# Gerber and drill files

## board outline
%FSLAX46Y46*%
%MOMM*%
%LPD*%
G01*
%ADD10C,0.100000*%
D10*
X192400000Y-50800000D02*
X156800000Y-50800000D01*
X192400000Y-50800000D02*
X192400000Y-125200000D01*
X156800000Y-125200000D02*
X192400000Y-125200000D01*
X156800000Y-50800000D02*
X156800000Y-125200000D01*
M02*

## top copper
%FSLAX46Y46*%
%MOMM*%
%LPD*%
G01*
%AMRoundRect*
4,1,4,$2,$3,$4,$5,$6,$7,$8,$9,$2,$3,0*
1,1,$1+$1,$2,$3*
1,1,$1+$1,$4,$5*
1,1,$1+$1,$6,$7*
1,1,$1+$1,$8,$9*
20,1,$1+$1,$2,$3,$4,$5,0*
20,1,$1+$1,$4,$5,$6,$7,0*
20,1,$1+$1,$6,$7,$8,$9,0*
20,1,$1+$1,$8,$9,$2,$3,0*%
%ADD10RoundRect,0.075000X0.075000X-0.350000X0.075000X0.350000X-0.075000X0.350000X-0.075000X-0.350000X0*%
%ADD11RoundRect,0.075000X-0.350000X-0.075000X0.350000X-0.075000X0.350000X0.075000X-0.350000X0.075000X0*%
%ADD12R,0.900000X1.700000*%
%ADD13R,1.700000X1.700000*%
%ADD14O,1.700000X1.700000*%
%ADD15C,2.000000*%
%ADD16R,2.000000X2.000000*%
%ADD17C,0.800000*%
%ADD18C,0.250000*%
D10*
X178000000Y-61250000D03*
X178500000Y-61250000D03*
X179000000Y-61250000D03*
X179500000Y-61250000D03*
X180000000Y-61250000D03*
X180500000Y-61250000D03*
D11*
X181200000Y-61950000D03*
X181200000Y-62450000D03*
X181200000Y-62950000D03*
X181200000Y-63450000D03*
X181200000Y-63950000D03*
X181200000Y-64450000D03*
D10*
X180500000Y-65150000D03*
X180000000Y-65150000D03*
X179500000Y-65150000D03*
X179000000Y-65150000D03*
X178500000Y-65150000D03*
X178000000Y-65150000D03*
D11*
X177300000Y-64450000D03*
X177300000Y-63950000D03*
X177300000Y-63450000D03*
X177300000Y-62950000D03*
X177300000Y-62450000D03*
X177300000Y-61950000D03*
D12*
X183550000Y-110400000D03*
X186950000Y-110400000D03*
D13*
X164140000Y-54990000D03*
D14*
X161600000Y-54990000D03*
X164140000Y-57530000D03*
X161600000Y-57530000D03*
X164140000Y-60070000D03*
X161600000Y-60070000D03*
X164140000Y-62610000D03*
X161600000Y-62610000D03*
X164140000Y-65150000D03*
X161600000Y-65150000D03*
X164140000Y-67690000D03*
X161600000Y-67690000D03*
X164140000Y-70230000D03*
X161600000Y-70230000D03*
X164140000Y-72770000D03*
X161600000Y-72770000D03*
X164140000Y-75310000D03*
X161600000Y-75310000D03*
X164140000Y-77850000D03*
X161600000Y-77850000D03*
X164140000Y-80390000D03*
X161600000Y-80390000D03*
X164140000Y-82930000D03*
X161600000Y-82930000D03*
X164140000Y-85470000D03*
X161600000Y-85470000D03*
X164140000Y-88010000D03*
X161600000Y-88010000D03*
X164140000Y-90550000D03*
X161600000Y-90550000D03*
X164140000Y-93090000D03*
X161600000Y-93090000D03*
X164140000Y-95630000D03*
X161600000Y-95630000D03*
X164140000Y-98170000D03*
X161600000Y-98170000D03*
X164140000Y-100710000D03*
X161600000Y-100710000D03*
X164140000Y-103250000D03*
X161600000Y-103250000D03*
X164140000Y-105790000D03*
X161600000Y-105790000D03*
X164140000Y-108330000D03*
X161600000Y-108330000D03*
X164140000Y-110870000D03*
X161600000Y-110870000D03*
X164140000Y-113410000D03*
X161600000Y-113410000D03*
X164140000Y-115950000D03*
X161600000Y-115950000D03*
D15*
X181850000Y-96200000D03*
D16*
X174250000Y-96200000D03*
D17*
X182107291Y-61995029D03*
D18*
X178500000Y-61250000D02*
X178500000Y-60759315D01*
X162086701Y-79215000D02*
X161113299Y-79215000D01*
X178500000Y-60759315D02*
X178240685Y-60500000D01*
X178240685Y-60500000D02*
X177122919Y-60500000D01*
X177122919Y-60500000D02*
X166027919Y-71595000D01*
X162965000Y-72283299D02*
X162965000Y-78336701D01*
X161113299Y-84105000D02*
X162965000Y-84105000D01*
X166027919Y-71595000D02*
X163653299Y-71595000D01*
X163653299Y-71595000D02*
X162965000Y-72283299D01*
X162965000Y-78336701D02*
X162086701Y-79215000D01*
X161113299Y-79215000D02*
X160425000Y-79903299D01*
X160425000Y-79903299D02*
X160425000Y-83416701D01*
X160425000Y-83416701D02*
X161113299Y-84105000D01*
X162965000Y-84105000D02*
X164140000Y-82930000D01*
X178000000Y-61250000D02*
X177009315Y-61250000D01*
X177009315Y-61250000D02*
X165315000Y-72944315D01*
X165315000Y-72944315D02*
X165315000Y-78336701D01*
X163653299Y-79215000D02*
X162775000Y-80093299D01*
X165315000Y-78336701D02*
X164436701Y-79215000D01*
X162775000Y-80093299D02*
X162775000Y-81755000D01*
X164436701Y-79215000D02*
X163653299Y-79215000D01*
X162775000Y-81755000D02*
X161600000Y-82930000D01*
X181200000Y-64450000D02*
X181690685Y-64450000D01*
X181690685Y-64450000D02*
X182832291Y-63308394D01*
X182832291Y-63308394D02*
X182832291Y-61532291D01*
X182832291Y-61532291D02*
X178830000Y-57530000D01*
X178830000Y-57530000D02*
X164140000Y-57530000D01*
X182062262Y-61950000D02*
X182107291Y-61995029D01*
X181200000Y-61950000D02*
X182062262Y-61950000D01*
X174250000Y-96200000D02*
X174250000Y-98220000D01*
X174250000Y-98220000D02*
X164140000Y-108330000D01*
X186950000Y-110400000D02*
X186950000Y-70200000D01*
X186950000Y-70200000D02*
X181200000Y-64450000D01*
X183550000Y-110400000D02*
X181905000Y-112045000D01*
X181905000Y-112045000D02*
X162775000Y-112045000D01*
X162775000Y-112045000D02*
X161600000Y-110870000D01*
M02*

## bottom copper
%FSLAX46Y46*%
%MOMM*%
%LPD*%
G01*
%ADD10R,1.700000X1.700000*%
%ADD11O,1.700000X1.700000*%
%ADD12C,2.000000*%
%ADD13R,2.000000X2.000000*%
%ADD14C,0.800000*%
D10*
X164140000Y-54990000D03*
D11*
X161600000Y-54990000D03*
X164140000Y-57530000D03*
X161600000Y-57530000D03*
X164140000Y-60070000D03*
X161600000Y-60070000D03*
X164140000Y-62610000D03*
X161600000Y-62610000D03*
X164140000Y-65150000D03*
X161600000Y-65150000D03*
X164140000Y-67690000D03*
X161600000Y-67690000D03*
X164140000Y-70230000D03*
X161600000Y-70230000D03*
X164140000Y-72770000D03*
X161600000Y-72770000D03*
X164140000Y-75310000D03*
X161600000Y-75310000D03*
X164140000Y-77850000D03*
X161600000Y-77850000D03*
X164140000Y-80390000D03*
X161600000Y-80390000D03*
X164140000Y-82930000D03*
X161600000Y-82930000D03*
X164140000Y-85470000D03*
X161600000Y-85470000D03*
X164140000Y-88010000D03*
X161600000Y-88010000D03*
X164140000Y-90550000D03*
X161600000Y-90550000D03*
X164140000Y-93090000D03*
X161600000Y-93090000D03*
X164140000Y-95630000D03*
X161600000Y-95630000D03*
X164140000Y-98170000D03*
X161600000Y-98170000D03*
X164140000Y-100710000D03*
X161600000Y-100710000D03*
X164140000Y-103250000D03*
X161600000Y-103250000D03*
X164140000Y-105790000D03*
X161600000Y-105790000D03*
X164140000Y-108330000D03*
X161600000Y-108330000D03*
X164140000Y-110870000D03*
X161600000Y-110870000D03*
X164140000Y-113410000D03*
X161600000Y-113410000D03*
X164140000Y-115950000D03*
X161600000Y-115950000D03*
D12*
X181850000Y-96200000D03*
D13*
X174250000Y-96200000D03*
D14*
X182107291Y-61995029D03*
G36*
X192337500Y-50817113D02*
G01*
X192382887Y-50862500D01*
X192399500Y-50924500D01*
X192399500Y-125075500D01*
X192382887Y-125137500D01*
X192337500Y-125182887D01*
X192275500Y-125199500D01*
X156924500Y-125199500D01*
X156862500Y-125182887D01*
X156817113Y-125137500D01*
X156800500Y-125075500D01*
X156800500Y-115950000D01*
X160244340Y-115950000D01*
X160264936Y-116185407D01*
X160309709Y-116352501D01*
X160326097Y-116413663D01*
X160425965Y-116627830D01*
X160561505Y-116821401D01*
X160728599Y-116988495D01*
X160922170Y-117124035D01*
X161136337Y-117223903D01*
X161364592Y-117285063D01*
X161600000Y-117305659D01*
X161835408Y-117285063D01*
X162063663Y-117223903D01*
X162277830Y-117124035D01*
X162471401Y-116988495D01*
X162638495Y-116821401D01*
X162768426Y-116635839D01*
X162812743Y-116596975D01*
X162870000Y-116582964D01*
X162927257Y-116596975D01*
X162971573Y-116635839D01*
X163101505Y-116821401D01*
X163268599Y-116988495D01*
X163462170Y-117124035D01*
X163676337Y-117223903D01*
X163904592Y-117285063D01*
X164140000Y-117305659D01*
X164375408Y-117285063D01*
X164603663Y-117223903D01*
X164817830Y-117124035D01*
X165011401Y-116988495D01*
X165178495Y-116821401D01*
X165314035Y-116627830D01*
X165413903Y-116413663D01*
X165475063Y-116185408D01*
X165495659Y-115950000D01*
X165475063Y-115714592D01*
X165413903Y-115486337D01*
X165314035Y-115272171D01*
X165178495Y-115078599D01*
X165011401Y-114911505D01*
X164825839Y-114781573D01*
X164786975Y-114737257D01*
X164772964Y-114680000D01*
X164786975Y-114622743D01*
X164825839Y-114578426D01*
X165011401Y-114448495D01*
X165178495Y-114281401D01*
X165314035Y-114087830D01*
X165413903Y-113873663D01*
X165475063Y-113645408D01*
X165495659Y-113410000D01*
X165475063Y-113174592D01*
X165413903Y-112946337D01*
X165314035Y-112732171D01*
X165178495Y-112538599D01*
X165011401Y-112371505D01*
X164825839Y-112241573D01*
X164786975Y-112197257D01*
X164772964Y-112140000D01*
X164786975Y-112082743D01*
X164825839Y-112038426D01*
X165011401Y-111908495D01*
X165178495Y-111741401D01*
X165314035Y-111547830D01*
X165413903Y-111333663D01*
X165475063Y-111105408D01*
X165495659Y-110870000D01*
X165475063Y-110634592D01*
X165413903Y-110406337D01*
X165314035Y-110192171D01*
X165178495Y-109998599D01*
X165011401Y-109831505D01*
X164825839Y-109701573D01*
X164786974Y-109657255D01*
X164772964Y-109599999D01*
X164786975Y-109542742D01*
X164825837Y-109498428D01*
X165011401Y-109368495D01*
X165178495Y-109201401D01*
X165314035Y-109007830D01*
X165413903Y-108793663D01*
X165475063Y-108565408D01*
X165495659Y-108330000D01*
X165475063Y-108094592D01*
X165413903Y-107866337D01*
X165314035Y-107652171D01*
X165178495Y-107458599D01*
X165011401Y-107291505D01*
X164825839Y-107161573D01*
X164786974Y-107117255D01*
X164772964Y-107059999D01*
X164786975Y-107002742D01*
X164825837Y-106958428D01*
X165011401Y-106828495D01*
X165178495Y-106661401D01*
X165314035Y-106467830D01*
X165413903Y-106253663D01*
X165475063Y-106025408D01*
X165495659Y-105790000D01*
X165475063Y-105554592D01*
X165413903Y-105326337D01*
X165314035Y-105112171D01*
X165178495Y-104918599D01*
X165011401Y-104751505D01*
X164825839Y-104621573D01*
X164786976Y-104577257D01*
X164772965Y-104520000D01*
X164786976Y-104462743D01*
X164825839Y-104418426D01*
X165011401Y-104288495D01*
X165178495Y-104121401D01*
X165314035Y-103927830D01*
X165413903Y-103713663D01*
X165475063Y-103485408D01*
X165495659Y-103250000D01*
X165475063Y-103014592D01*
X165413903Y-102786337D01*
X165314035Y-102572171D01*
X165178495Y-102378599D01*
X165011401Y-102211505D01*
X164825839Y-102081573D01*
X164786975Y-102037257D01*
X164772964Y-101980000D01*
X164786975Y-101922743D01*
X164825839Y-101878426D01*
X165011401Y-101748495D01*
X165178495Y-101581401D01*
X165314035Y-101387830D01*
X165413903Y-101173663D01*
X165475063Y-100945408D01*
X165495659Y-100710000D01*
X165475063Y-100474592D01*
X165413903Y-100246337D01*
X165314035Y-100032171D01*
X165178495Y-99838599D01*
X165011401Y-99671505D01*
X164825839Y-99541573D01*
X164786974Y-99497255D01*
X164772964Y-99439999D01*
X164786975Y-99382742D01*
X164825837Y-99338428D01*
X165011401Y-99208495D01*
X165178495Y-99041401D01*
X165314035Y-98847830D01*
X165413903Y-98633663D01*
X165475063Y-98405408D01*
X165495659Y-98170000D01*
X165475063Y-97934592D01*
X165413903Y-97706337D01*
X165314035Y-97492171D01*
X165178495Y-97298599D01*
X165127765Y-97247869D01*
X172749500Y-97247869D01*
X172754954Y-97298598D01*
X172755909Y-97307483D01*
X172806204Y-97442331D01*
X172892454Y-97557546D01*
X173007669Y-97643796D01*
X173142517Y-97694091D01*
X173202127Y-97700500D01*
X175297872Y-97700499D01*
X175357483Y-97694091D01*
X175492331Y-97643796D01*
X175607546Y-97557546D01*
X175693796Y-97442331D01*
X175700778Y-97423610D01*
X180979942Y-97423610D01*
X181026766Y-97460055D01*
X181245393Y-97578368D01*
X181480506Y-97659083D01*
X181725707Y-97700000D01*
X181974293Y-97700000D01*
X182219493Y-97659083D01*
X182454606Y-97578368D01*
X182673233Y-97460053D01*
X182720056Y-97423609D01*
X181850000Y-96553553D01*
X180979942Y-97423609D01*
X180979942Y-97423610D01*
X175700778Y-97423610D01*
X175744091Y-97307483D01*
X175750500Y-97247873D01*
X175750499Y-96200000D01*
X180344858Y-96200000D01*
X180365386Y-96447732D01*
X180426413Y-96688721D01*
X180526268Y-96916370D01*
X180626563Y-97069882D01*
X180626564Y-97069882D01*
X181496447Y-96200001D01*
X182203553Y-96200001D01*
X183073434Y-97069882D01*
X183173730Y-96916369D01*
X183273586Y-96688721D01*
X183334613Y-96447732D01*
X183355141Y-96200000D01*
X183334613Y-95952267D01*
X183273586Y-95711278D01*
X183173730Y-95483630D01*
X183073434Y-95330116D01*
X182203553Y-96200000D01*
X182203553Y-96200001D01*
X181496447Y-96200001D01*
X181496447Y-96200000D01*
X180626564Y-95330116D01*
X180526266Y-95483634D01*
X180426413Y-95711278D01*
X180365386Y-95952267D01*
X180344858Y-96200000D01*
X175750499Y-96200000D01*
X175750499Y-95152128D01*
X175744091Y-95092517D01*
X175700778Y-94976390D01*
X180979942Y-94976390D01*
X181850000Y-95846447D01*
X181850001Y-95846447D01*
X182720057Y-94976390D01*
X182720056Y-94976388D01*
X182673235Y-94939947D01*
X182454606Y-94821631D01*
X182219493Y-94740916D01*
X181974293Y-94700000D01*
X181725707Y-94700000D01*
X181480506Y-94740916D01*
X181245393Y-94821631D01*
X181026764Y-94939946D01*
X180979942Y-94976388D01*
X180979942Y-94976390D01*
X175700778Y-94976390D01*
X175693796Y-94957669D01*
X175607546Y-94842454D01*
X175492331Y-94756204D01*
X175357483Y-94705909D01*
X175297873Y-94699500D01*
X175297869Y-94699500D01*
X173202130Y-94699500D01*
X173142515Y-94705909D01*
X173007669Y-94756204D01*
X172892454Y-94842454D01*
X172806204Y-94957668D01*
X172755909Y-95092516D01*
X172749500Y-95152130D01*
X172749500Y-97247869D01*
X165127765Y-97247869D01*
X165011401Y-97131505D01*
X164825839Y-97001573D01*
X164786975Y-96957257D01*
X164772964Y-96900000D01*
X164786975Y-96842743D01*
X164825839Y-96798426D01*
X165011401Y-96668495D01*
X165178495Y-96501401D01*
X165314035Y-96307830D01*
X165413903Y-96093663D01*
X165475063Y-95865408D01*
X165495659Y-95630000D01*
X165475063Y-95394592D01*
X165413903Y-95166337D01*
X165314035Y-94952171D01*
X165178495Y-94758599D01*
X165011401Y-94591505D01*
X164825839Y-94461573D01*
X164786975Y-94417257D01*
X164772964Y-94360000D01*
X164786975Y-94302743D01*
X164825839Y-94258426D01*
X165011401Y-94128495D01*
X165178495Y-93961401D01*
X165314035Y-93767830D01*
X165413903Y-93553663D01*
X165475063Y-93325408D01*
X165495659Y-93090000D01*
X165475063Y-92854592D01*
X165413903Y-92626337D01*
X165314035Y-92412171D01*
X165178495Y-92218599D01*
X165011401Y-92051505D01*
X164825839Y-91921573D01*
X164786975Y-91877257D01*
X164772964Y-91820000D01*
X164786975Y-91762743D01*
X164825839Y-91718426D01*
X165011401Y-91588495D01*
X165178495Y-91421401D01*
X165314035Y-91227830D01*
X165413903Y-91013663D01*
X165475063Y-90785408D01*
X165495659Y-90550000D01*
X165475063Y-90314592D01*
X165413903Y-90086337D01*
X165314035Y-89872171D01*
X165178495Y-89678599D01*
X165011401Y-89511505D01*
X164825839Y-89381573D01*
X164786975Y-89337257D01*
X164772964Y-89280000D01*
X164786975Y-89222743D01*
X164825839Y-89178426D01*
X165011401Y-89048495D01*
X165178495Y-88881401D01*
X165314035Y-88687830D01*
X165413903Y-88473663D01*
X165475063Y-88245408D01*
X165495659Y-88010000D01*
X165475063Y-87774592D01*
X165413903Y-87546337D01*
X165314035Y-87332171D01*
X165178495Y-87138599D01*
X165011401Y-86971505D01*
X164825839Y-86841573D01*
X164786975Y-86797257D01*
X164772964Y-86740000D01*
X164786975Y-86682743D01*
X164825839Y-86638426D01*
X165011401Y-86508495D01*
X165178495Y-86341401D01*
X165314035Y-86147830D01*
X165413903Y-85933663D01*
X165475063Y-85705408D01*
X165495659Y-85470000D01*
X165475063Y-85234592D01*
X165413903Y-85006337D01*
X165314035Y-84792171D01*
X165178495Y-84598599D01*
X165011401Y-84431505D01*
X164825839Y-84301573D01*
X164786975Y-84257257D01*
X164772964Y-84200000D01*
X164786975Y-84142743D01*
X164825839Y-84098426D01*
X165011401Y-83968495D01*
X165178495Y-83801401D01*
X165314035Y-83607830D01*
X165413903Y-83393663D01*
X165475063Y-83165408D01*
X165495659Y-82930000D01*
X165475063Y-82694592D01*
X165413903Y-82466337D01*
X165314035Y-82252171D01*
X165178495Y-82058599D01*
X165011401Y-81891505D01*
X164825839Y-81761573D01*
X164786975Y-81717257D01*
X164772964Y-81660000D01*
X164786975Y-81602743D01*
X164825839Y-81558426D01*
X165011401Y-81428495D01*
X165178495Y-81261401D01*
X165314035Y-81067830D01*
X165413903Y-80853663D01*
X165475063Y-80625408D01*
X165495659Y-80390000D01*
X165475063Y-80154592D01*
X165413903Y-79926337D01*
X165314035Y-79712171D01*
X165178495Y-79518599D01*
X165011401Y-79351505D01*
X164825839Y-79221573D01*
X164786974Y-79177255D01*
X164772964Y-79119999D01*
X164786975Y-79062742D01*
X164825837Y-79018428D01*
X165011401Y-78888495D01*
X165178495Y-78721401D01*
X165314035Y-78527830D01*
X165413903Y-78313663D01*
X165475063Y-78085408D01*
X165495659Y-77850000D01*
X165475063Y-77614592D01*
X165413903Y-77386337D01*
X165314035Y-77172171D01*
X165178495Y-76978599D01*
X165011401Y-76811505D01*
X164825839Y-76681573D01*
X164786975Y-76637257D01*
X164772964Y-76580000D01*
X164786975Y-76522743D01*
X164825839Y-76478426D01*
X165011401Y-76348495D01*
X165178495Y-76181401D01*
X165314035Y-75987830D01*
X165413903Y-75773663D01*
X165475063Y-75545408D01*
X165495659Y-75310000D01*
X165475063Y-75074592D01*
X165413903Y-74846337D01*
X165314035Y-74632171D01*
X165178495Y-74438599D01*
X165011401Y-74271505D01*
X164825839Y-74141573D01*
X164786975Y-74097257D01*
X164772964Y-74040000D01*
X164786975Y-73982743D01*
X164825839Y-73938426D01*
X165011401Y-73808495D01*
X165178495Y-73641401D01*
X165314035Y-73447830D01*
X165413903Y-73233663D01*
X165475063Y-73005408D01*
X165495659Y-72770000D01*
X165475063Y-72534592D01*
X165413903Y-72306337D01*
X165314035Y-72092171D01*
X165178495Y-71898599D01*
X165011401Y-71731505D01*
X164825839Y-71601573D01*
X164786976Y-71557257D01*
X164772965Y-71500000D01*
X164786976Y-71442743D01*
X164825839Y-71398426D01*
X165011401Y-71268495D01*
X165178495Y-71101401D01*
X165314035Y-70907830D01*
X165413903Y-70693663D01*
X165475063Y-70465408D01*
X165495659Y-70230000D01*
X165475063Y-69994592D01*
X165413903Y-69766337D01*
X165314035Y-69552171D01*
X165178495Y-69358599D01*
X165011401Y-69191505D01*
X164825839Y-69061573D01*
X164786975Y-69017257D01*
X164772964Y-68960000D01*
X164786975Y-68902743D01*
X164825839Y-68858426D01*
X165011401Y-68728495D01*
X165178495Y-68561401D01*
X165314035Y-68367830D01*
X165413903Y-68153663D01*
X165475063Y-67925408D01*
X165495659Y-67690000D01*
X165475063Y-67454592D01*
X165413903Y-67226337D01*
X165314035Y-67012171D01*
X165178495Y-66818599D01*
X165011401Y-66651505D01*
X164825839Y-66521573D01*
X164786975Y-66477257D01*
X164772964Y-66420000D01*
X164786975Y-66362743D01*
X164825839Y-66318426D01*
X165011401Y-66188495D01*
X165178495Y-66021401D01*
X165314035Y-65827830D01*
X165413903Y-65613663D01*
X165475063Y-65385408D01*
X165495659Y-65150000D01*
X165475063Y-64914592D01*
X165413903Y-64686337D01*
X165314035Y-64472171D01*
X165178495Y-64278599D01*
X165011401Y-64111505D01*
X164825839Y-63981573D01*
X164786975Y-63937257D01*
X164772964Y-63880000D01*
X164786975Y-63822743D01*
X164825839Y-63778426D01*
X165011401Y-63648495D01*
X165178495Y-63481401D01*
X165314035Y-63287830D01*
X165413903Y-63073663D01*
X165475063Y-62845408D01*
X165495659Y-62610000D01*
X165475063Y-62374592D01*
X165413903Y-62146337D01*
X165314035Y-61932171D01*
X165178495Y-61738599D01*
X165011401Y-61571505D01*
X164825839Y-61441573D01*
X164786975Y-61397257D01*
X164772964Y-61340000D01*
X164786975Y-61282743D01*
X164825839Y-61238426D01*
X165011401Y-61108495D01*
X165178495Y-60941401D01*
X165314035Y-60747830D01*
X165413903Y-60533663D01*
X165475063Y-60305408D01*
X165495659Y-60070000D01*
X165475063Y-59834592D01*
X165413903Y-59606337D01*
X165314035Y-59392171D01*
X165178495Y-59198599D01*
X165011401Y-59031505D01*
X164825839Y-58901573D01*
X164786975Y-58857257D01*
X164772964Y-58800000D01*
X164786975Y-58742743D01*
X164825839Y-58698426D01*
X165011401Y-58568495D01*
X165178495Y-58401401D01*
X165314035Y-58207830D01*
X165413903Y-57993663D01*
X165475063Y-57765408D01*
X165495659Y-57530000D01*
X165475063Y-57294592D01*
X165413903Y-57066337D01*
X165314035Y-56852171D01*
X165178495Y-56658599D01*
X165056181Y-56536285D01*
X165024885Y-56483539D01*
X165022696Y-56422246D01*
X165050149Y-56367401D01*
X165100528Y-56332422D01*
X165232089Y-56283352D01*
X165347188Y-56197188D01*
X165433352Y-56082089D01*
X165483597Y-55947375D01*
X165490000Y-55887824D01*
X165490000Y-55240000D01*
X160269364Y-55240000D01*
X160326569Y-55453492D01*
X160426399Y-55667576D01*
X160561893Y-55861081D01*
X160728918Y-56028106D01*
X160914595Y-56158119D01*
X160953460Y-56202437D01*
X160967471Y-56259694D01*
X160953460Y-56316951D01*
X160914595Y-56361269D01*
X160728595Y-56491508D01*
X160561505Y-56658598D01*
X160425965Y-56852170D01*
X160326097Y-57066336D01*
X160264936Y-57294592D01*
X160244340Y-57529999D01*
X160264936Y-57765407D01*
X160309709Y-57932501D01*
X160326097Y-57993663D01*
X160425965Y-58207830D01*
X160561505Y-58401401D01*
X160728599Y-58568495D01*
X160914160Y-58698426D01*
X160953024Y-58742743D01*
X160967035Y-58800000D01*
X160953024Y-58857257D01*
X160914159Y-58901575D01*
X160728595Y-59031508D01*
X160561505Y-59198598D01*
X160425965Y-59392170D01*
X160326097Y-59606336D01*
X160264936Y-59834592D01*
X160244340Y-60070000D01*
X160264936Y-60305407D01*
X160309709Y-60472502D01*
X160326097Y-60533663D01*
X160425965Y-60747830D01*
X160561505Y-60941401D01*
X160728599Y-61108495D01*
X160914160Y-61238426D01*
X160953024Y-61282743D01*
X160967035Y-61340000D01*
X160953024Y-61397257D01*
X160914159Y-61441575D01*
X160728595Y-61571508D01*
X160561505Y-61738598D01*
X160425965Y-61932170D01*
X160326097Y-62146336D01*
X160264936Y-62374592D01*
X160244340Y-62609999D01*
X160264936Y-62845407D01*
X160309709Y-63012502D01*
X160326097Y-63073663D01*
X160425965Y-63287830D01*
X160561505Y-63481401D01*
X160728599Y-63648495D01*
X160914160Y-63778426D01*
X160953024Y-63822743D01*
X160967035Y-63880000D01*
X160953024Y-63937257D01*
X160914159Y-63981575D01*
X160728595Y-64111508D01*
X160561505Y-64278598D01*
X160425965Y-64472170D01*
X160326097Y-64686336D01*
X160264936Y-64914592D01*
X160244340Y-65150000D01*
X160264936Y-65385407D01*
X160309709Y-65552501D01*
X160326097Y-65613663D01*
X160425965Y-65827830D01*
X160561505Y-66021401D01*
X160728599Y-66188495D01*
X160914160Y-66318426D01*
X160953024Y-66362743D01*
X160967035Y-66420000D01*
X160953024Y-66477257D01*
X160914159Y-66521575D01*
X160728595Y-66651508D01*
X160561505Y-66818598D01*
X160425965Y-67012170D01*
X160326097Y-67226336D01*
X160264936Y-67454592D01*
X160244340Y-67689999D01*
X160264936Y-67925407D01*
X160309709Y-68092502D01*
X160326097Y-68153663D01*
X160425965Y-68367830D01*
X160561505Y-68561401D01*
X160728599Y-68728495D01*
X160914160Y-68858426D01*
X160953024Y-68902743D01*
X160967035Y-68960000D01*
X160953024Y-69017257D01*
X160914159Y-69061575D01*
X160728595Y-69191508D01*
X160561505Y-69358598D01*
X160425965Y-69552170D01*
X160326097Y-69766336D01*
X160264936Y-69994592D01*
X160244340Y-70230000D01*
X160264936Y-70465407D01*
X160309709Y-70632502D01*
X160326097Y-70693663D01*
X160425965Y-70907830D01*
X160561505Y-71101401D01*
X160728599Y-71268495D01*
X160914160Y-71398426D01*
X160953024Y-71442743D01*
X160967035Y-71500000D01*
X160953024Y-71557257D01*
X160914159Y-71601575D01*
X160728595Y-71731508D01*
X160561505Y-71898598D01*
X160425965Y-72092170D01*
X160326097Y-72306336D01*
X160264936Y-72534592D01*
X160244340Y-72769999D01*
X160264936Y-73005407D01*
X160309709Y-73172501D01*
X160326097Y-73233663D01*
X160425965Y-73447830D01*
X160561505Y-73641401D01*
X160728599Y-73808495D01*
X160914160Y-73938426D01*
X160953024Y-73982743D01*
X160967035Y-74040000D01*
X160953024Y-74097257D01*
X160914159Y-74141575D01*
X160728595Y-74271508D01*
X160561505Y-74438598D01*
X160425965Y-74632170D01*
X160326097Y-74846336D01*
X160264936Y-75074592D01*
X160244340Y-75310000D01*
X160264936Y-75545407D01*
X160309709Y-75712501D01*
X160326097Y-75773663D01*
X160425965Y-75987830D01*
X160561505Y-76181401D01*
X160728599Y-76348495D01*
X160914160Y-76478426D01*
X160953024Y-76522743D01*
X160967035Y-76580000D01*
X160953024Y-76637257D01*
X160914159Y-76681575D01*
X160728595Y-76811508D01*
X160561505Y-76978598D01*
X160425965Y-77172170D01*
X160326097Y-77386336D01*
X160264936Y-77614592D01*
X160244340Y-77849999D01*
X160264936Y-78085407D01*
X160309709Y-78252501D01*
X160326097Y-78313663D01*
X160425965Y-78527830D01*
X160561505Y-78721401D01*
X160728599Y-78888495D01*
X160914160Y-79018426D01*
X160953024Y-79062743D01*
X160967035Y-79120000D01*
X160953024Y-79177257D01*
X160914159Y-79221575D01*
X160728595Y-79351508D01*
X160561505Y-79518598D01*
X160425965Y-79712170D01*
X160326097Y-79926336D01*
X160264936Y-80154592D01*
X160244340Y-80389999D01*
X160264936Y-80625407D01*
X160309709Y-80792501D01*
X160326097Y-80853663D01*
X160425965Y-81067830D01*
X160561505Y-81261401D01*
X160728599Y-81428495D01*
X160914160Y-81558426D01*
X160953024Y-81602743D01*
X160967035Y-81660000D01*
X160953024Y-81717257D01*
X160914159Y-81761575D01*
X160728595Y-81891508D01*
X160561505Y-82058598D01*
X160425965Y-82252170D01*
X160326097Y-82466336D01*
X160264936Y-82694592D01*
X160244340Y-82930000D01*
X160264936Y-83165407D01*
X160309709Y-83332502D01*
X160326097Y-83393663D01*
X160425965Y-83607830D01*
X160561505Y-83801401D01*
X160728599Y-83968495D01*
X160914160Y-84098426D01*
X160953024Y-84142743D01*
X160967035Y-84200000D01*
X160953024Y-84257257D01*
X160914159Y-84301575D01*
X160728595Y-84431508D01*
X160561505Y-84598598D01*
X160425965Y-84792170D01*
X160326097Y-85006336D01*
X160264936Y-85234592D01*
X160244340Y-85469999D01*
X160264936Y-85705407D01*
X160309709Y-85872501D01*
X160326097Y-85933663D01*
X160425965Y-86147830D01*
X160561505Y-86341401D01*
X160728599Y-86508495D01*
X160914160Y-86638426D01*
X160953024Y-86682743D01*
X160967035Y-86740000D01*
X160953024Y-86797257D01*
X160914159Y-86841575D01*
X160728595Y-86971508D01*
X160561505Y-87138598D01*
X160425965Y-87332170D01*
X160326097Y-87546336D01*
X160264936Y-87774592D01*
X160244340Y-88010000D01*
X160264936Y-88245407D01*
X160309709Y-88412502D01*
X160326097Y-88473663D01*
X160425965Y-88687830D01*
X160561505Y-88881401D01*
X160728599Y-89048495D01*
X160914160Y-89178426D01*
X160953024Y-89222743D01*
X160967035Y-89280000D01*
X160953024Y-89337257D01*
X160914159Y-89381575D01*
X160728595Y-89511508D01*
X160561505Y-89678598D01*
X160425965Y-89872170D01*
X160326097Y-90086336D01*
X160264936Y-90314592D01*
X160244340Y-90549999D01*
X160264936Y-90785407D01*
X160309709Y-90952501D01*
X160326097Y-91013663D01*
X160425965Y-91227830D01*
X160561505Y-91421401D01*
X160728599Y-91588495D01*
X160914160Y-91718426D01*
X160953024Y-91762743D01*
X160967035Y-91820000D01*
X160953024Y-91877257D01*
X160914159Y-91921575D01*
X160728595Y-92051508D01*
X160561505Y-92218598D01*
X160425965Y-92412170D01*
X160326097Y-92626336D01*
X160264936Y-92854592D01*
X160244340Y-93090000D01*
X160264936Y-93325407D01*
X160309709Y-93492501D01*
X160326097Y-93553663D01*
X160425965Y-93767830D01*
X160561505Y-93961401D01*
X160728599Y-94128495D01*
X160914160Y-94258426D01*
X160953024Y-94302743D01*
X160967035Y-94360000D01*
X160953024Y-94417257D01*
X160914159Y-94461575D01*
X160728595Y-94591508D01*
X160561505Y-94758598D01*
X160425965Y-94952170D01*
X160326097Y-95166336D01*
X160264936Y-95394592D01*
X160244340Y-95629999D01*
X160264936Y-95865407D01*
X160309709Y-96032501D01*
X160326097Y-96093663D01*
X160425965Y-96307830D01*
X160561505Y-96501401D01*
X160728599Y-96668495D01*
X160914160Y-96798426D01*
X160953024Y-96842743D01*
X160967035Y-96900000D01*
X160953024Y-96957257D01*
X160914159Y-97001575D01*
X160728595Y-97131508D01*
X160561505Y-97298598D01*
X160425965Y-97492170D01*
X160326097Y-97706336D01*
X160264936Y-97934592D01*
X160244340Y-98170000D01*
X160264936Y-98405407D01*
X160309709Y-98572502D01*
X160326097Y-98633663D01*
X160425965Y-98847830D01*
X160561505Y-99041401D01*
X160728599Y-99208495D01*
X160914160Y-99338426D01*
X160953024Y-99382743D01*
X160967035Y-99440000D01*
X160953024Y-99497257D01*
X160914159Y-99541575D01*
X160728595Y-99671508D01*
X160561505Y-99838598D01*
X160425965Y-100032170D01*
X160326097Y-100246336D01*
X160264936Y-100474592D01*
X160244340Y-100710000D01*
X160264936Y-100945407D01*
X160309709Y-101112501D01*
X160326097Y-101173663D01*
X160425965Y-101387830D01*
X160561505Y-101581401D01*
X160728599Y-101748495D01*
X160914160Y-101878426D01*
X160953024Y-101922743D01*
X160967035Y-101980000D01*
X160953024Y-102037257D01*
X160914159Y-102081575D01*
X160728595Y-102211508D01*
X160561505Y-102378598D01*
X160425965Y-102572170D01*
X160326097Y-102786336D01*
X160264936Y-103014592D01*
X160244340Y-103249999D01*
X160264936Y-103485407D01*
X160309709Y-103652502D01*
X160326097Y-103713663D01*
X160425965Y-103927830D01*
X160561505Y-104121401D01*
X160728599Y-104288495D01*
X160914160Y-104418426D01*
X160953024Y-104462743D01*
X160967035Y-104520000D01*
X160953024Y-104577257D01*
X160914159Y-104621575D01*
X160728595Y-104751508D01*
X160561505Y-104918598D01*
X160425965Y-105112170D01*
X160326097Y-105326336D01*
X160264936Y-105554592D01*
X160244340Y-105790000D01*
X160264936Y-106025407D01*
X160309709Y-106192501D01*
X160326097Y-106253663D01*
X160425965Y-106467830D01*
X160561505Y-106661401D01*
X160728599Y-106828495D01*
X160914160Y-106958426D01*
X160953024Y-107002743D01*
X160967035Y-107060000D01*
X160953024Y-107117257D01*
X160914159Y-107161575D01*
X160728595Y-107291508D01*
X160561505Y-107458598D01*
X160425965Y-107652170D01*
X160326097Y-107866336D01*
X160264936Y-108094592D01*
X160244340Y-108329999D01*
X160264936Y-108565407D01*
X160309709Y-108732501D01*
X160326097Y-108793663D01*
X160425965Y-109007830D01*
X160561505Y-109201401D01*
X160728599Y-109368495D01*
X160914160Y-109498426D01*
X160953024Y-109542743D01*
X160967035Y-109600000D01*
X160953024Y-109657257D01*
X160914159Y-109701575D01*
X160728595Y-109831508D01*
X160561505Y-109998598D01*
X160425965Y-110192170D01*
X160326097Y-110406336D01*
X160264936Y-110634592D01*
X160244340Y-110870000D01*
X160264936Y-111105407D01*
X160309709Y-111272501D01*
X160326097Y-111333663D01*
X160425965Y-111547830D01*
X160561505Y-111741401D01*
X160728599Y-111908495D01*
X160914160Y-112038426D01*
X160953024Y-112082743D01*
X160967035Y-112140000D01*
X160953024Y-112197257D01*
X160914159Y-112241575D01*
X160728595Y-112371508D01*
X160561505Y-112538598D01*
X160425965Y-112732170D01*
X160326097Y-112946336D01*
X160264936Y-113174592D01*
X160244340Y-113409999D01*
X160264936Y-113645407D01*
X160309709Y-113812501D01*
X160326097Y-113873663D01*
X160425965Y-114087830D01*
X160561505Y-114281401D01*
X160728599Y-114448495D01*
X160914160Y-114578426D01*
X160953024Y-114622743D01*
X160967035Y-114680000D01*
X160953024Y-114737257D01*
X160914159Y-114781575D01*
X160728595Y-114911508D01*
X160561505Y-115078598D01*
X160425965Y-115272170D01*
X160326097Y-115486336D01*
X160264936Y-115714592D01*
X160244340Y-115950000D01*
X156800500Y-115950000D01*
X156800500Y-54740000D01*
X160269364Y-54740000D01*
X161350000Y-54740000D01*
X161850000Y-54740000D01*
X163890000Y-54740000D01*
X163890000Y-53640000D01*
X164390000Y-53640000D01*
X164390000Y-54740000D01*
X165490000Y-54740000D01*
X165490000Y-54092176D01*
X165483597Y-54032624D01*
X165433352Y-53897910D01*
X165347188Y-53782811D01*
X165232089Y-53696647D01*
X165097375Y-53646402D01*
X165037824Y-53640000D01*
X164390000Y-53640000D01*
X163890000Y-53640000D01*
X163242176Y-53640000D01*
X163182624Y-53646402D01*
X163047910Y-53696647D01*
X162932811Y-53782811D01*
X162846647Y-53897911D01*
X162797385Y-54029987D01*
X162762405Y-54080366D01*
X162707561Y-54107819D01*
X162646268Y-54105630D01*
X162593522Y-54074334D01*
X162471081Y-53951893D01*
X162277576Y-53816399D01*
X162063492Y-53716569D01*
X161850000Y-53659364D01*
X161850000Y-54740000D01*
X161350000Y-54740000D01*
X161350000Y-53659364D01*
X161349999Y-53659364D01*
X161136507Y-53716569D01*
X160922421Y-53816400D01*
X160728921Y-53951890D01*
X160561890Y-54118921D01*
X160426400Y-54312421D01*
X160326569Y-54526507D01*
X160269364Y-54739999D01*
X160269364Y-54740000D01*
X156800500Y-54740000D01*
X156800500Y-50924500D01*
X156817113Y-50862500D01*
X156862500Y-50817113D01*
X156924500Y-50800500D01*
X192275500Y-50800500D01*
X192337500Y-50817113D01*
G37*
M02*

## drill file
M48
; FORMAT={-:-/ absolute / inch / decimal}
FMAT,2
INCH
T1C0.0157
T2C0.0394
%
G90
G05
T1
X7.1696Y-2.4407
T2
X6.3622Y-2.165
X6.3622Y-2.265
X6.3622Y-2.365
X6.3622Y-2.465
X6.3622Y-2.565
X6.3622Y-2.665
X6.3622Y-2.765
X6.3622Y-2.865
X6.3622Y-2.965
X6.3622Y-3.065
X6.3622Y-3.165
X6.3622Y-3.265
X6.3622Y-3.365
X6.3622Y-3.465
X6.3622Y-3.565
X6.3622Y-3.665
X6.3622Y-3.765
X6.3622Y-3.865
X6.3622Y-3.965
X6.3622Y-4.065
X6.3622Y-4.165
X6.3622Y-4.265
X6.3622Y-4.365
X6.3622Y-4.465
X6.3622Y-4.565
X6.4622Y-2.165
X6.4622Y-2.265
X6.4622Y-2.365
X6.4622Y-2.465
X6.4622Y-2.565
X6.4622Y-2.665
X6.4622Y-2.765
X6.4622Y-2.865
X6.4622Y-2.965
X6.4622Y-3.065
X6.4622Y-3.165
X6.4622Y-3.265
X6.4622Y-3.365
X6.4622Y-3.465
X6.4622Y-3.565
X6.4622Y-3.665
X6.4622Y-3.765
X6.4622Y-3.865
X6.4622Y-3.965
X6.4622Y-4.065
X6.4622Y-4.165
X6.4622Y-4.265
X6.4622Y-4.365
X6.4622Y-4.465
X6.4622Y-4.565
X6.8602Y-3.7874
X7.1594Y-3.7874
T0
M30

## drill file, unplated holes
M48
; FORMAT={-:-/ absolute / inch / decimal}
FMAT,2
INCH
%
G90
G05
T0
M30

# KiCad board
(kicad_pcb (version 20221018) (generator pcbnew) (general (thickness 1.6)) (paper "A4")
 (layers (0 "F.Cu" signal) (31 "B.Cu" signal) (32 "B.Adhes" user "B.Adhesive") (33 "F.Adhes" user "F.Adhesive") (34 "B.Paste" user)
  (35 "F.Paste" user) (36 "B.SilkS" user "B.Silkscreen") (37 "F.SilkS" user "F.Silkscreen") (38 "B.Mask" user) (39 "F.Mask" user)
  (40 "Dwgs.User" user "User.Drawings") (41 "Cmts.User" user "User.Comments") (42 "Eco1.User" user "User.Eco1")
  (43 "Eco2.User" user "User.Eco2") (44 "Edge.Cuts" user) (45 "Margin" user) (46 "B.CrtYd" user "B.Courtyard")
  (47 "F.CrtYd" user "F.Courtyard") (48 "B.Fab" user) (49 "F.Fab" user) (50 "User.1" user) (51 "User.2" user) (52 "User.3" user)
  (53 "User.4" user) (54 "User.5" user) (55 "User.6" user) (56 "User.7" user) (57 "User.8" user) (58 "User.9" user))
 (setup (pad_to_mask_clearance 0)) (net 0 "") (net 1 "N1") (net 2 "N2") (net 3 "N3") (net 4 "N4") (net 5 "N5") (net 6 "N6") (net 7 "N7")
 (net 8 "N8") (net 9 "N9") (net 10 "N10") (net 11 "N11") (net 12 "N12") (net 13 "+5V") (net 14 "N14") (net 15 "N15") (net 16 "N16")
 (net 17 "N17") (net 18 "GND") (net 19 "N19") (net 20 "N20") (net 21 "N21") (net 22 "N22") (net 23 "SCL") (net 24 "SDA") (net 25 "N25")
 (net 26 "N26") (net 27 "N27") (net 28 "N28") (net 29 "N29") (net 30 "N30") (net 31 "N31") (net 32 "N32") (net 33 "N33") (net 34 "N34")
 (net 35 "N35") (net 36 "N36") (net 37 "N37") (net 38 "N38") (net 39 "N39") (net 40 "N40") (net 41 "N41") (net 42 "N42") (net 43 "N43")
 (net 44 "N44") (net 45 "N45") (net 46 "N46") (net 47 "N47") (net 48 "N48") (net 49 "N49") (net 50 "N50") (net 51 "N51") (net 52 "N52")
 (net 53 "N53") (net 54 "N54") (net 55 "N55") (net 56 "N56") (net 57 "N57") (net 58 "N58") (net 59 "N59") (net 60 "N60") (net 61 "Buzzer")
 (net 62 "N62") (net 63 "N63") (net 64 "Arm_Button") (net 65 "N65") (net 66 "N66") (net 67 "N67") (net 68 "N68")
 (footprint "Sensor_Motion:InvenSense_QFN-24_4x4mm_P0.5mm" (layer "F.Cu") (at 179.25 63.2)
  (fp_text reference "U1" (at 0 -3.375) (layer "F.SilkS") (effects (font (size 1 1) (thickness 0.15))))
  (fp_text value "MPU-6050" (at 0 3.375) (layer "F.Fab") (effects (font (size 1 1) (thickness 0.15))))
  (pad "1" smd roundrect (at -1.95 -1.25) (size 0.85 0.3) (layers "F.Cu" "F.Paste" "F.Mask") (roundrect_rratio 0.25) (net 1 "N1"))
  (pad "2" smd roundrect (at -1.95 -0.75) (size 0.85 0.3) (layers "F.Cu" "F.Paste" "F.Mask") (roundrect_rratio 0.25) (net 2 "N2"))
  (pad "3" smd roundrect (at -1.95 -0.25) (size 0.85 0.3) (layers "F.Cu" "F.Paste" "F.Mask") (roundrect_rratio 0.25) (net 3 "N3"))
  (pad "4" smd roundrect (at -1.95 0.25) (size 0.85 0.3) (layers "F.Cu" "F.Paste" "F.Mask") (roundrect_rratio 0.25) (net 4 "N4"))
  (pad "5" smd roundrect (at -1.95 0.75) (size 0.85 0.3) (layers "F.Cu" "F.Paste" "F.Mask") (roundrect_rratio 0.25) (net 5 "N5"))
  (pad "6" smd roundrect (at -1.95 1.25) (size 0.85 0.3) (layers "F.Cu" "F.Paste" "F.Mask") (roundrect_rratio 0.25) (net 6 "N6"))
  (pad "7" smd roundrect (at -1.25 1.95 90) (size 0.85 0.3) (layers "F.Cu" "F.Paste" "F.Mask") (roundrect_rratio 0.25) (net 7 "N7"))
  (pad "8" smd roundrect (at -0.75 1.95 90) (size 0.85 0.3) (layers "F.Cu" "F.Paste" "F.Mask") (roundrect_rratio 0.25) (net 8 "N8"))
  (pad "9" smd roundrect (at -0.25 1.95 90) (size 0.85 0.3) (layers "F.Cu" "F.Paste" "F.Mask") (roundrect_rratio 0.25) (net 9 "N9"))
  (pad "10" smd roundrect (at 0.25 1.95 90) (size 0.85 0.3) (layers "F.Cu" "F.Paste" "F.Mask") (roundrect_rratio 0.25) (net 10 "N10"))
  (pad "11" smd roundrect (at 0.75 1.95 90) (size 0.85 0.3) (layers "F.Cu" "F.Paste" "F.Mask") (roundrect_rratio 0.25) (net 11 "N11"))
  (pad "12" smd roundrect (at 1.25 1.95 90) (size 0.85 0.3) (layers "F.Cu" "F.Paste" "F.Mask") (roundrect_rratio 0.25) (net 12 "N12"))
  (pad "13" smd roundrect (at 1.95 1.25) (size 0.85 0.3) (layers "F.Cu" "F.Paste" "F.Mask") (roundrect_rratio 0.25) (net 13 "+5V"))
  (pad "14" smd roundrect (at 1.95 0.75) (size 0.85 0.3) (layers "F.Cu" "F.Paste" "F.Mask") (roundrect_rratio 0.25) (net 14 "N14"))
  (pad "15" smd roundrect (at 1.95 0.25) (size 0.85 0.3) (layers "F.Cu" "F.Paste" "F.Mask") (roundrect_rratio 0.25) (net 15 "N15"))
  (pad "16" smd roundrect (at 1.95 -0.25) (size 0.85 0.3) (layers "F.Cu" "F.Paste" "F.Mask") (roundrect_rratio 0.25) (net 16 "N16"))
  (pad "17" smd roundrect (at 1.95 -0.75) (size 0.85 0.3) (layers "F.Cu" "F.Paste" "F.Mask") (roundrect_rratio 0.25) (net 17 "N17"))
  (pad "18" smd roundrect (at 1.95 -1.25) (size 0.85 0.3) (layers "F.Cu" "F.Paste" "F.Mask") (roundrect_rratio 0.25) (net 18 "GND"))
  (pad "19" smd roundrect (at 1.25 -1.95 90) (size 0.85 0.3) (layers "F.Cu" "F.Paste" "F.Mask") (roundrect_rratio 0.25) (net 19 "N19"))
  (pad "20" smd roundrect (at 0.75 -1.95 90) (size 0.85 0.3) (layers "F.Cu" "F.Paste" "F.Mask") (roundrect_rratio 0.25) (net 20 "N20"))
  (pad "21" smd roundrect (at 0.25 -1.95 90) (size 0.85 0.3) (layers "F.Cu" "F.Paste" "F.Mask") (roundrect_rratio 0.25) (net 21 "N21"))
  (pad "22" smd roundrect (at -0.25 -1.95 90) (size 0.85 0.3) (layers "F.Cu" "F.Paste" "F.Mask") (roundrect_rratio 0.25) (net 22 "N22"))
  (pad "23" smd roundrect (at -0.75 -1.95 90) (size 0.85 0.3) (layers "F.Cu" "F.Paste" "F.Mask") (roundrect_rratio 0.25) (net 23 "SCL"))
  (pad "24" smd roundrect (at -1.25 -1.95 90) (size 0.85 0.3) (layers "F.Cu" "F.Paste" "F.Mask") (roundrect_rratio 0.25) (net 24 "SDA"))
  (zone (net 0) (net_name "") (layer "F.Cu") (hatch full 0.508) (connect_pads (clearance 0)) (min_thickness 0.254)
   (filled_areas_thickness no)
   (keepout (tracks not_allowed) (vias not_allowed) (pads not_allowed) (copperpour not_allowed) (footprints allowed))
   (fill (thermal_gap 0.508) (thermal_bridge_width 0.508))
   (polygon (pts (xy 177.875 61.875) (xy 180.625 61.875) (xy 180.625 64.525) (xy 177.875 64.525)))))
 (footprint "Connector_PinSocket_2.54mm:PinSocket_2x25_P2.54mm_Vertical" (layer "F.Cu") (at 164.14 54.99)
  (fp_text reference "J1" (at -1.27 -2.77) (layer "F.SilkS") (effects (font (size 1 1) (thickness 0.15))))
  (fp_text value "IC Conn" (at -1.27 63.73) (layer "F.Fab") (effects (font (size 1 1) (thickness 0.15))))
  (pad "1" thru_hole rect (at 0 0) (size 1.7 1.7) (drill 1) (layers "*.Cu" "*.Mask") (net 18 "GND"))
  (pad "2" thru_hole oval (at -2.54 0) (size 1.7 1.7) (drill 1) (layers "*.Cu" "*.Mask") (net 18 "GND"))
  (pad "3" thru_hole oval (at 0 2.54) (size 1.7 1.7) (drill 1) (layers "*.Cu" "*.Mask") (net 13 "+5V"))
  (pad "4" thru_hole oval (at -2.54 2.54) (size 1.7 1.7) (drill 1) (layers "*.Cu" "*.Mask") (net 13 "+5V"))
  (pad "5" thru_hole oval (at 0 5.08) (size 1.7 1.7) (drill 1) (layers "*.Cu" "*.Mask") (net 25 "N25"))
  (pad "6" thru_hole oval (at -2.54 5.08) (size 1.7 1.7) (drill 1) (layers "*.Cu" "*.Mask") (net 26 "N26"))
  (pad "7" thru_hole oval (at 0 7.62) (size 1.7 1.7) (drill 1) (layers "*.Cu" "*.Mask") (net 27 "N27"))
  (pad "8" thru_hole oval (at -2.54 7.62) (size 1.7 1.7) (drill 1) (layers "*.Cu" "*.Mask") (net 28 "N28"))
  (pad "9" thru_hole oval (at 0 10.16) (size 1.7 1.7) (drill 1) (layers "*.Cu" "*.Mask") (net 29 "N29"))
  (pad "10" thru_hole oval (at -2.54 10.16) (size 1.7 1.7) (drill 1) (layers "*.Cu" "*.Mask") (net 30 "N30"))
  (pad "11" thru_hole oval (at 0 12.7) (size 1.7 1.7) (drill 1) (layers "*.Cu" "*.Mask") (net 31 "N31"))
  (pad "12" thru_hole oval (at -2.54 12.7) (size 1.7 1.7) (drill 1) (layers "*.Cu" "*.Mask") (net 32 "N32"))
  (pad "13" thru_hole oval (at 0 15.24) (size 1.7 1.7) (drill 1) (layers "*.Cu" "*.Mask") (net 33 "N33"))
  (pad "14" thru_hole oval (at -2.54 15.24) (size 1.7 1.7) (drill 1) (layers "*.Cu" "*.Mask") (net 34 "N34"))
  (pad "15" thru_hole oval (at 0 17.78) (size 1.7 1.7) (drill 1) (layers "*.Cu" "*.Mask") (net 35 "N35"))
  (pad "16" thru_hole oval (at -2.54 17.78) (size 1.7 1.7) (drill 1) (layers "*.Cu" "*.Mask") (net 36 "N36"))
  (pad "17" thru_hole oval (at 0 20.32) (size 1.7 1.7) (drill 1) (layers "*.Cu" "*.Mask") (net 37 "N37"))
  (pad "18" thru_hole oval (at -2.54 20.32) (size 1.7 1.7) (drill 1) (layers "*.Cu" "*.Mask") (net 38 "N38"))
  (pad "19" thru_hole oval (at 0 22.86) (size 1.7 1.7) (drill 1) (layers "*.Cu" "*.Mask") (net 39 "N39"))
  (pad "20" thru_hole oval (at -2.54 22.86) (size 1.7 1.7) (drill 1) (layers "*.Cu" "*.Mask") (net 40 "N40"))
  (pad "21" thru_hole oval (at 0 25.4) (size 1.7 1.7) (drill 1) (layers "*.Cu" "*.Mask") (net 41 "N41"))
  (pad "22" thru_hole oval (at -2.54 25.4) (size 1.7 1.7) (drill 1) (layers "*.Cu" "*.Mask") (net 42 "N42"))
  (pad "23" thru_hole oval (at 0 27.94) (size 1.7 1.7) (drill 1) (layers "*.Cu" "*.Mask") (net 23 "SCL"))
  (pad "24" thru_hole oval (at -2.54 27.94) (size 1.7 1.7) (drill 1) (layers "*.Cu" "*.Mask") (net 24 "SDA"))
  (pad "25" thru_hole oval (at 0 30.48) (size 1.7 1.7) (drill 1) (layers "*.Cu" "*.Mask") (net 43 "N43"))
  (pad "26" thru_hole oval (at -2.54 30.48) (size 1.7 1.7) (drill 1) (layers "*.Cu" "*.Mask") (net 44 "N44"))
  (pad "27" thru_hole oval (at 0 33.02) (size 1.7 1.7) (drill 1) (layers "*.Cu" "*.Mask") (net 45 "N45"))
  (pad "28" thru_hole oval (at -2.54 33.02) (size 1.7 1.7) (drill 1) (layers "*.Cu" "*.Mask") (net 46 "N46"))
  (pad "29" thru_hole oval (at 0 35.56) (size 1.7 1.7) (drill 1) (layers "*.Cu" "*.Mask") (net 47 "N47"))
  (pad "30" thru_hole oval (at -2.54 35.56) (size 1.7 1.7) (drill 1) (layers "*.Cu" "*.Mask") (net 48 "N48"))
  (pad "31" thru_hole oval (at 0 38.1) (size 1.7 1.7) (drill 1) (layers "*.Cu" "*.Mask") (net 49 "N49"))
  (pad "32" thru_hole oval (at -2.54 38.1) (size 1.7 1.7) (drill 1) (layers "*.Cu" "*.Mask") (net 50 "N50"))
  (pad "33" thru_hole oval (at 0 40.64) (size 1.7 1.7) (drill 1) (layers "*.Cu" "*.Mask") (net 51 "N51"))
  (pad "34" thru_hole oval (at -2.54 40.64) (size 1.7 1.7) (drill 1) (layers "*.Cu" "*.Mask") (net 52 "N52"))
  (pad "35" thru_hole oval (at 0 43.18) (size 1.7 1.7) (drill 1) (layers "*.Cu" "*.Mask") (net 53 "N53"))
  (pad "36" thru_hole oval (at -2.54 43.18) (size 1.7 1.7) (drill 1) (layers "*.Cu" "*.Mask") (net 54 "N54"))
  (pad "37" thru_hole oval (at 0 45.72) (size 1.7 1.7) (drill 1) (layers "*.Cu" "*.Mask") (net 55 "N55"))
  (pad "38" thru_hole oval (at -2.54 45.72) (size 1.7 1.7) (drill 1) (layers "*.Cu" "*.Mask") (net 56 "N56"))
  (pad "39" thru_hole oval (at 0 48.26) (size 1.7 1.7) (drill 1) (layers "*.Cu" "*.Mask") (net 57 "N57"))
  (pad "40" thru_hole oval (at -2.54 48.26) (size 1.7 1.7) (drill 1) (layers "*.Cu" "*.Mask") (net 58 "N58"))
  (pad "41" thru_hole oval (at 0 50.8) (size 1.7 1.7) (drill 1) (layers "*.Cu" "*.Mask") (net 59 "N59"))
  (pad "42" thru_hole oval (at -2.54 50.8) (size 1.7 1.7) (drill 1) (layers "*.Cu" "*.Mask") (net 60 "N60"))
  (pad "43" thru_hole oval (at 0 53.34) (size 1.7 1.7) (drill 1) (layers "*.Cu" "*.Mask") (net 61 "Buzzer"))
  (pad "44" thru_hole oval (at -2.54 53.34) (size 1.7 1.7) (drill 1) (layers "*.Cu" "*.Mask") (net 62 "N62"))
  (pad "45" thru_hole oval (at 0 55.88) (size 1.7 1.7) (drill 1) (layers "*.Cu" "*.Mask") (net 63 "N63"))
  (pad "46" thru_hole oval (at -2.54 55.88) (size 1.7 1.7) (drill 1) (layers "*.Cu" "*.Mask") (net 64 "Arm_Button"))
  (pad "47" thru_hole oval (at 0 58.42) (size 1.7 1.7) (drill 1) (layers "*.Cu" "*.Mask") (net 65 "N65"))
  (pad "48" thru_hole oval (at -2.54 58.42) (size 1.7 1.7) (drill 1) (layers "*.Cu" "*.Mask") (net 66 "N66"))
  (pad "49" thru_hole oval (at 0 60.96) (size 1.7 1.7) (drill 1) (layers "*.Cu" "*.Mask") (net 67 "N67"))
  (pad "50" thru_hole oval (at -2.54 60.96) (size 1.7 1.7) (drill 1) (layers "*.Cu" "*.Mask") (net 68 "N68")))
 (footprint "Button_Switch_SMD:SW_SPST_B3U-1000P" (layer "F.Cu") (at 185.25 110.4 180)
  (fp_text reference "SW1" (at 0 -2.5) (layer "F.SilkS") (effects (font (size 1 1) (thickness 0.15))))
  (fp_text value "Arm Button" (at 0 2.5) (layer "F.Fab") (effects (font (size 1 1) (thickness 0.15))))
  (pad "1" smd rect (at -1.7 0 180) (size 0.9 1.7) (layers "F.Cu" "F.Paste" "F.Mask") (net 13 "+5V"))
  (pad "2" smd rect (at 1.7 0 180) (size 0.9 1.7) (layers "F.Cu" "F.Paste" "F.Mask") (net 64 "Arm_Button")))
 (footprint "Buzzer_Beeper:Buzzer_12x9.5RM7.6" (layer "F.Cu") (at 174.25 96.2)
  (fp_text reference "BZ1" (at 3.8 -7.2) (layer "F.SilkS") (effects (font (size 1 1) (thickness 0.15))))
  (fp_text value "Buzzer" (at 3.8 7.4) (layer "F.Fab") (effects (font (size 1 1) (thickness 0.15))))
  (pad "1" thru_hole rect (at 0 0) (size 2 2) (drill 1) (layers "*.Cu" "*.Mask") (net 61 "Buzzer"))
  (pad "2" thru_hole circle (at 7.6 0) (size 2 2) (drill 1) (layers "*.Cu" "*.Mask") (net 18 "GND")))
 (gr_line (start 156.8 125.2) (end 192.4 125.2) (stroke (width 0.1) (type default)) (layer "Edge.Cuts"))
 (gr_line (start 192.4 50.8) (end 156.8 50.8) (stroke (width 0.1) (type default)) (layer "Edge.Cuts"))
 (gr_line (start 156.8 50.8) (end 156.8 125.2) (stroke (width 0.1) (type default)) (layer "Edge.Cuts"))
 (gr_line (start 192.4 50.8) (end 192.4 125.2) (stroke (width 0.1) (type default)) (layer "Edge.Cuts"))
 (segment (start 174.25 98.22) (end 164.14 108.33) (width 0.25) (layer "F.Cu") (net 61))
 (segment (start 174.25 96.2) (end 174.25 98.22) (width 0.25) (layer "F.Cu") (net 61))
 (segment (start 182.062262 61.95) (end 182.107291 61.995029) (width 0.25) (layer "F.Cu") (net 18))
 (segment (start 181.2 61.95) (end 182.062262 61.95) (width 0.25) (layer "F.Cu") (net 18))
 (via (at 182.107291 61.995029) (size 0.8) (drill 0.4) (layers "F.Cu" "B.Cu") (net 18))
 (segment (start 182.832291 63.308394) (end 182.832291 61.532291) (width 0.25) (layer "F.Cu") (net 13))
 (segment (start 178.83 57.53) (end 164.14 57.53) (width 0.25) (layer "F.Cu") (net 13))
 (segment (start 182.832291 61.532291) (end 178.83 57.53) (width 0.25) (layer "F.Cu") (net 13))
 (segment (start 181.690685 64.45) (end 182.832291 63.308394) (width 0.25) (layer "F.Cu") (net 13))
 (segment (start 181.2 64.45) (end 181.690685 64.45) (width 0.25) (layer "F.Cu") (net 13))
 (segment (start 186.95 110.4) (end 186.95 70.2) (width 0.25) (layer "F.Cu") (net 13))
 (segment (start 186.95 70.2) (end 181.2 64.45) (width 0.25) (layer "F.Cu") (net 13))
 (segment (start 162.965 72.283299) (end 162.965 78.336701) (width 0.25) (layer "F.Cu") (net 23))
 (segment (start 178.240685 60.5) (end 177.122919 60.5) (width 0.25) (layer "F.Cu") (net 23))
 (segment (start 161.113299 84.105) (end 162.965 84.105) (width 0.25) (layer "F.Cu") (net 23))
 (segment (start 178.5 61.25) (end 178.5 60.759315) (width 0.25) (layer "F.Cu") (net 23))
 (segment (start 163.653299 71.595) (end 162.965 72.283299) (width 0.25) (layer "F.Cu") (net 23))
 (segment (start 178.5 60.759315) (end 178.240685 60.5) (width 0.25) (layer "F.Cu") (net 23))
 (segment (start 160.425 83.416701) (end 161.113299 84.105) (width 0.25) (layer "F.Cu") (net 23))
 (segment (start 162.086701 79.215) (end 161.113299 79.215) (width 0.25) (layer "F.Cu") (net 23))
 (segment (start 162.965 84.105) (end 164.14 82.93) (width 0.25) (layer "F.Cu") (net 23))
 (segment (start 177.122919 60.5) (end 166.027919 71.595) (width 0.25) (layer "F.Cu") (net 23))
 (segment (start 162.965 78.336701) (end 162.086701 79.215) (width 0.25) (layer "F.Cu") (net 23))
 (segment (start 161.113299 79.215) (end 160.425 79.903299) (width 0.25) (layer "F.Cu") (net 23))
 (segment (start 160.425 79.903299) (end 160.425 83.416701) (width 0.25) (layer "F.Cu") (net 23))
 (segment (start 166.027919 71.595) (end 163.653299 71.595) (width 0.25) (layer "F.Cu") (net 23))
 (segment (start 165.315 78.336701) (end 164.436701 79.215) (width 0.25) (layer "F.Cu") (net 24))
 (segment (start 163.653299 79.215) (end 162.775 80.093299) (width 0.25) (layer "F.Cu") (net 24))
 (segment (start 178 61.25) (end 177.009315 61.25) (width 0.25) (layer "F.Cu") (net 24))
 (segment (start 164.436701 79.215) (end 163.653299 79.215) (width 0.25) (layer "F.Cu") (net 24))
 (segment (start 177.009315 61.25) (end 165.315 72.944315) (width 0.25) (layer "F.Cu") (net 24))
 (segment (start 162.775 81.755) (end 161.6 82.93) (width 0.25) (layer "F.Cu") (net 24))
 (segment (start 162.775 80.093299) (end 162.775 81.755) (width 0.25) (layer "F.Cu") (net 24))
 (segment (start 165.315 72.944315) (end 165.315 78.336701) (width 0.25) (layer "F.Cu") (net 24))
 (segment (start 181.905 112.045) (end 162.775 112.045) (width 0.25) (layer "F.Cu") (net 64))
 (segment (start 183.55 110.4) (end 181.905 112.045) (width 0.25) (layer "F.Cu") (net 64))
 (segment (start 162.775 112.045) (end 161.6 110.87) (width 0.25) (layer "F.Cu") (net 64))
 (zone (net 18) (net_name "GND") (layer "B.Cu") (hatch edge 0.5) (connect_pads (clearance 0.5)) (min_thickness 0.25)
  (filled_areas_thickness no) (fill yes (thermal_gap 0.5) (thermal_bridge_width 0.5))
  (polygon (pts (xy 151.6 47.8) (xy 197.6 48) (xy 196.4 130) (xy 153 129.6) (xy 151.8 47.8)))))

